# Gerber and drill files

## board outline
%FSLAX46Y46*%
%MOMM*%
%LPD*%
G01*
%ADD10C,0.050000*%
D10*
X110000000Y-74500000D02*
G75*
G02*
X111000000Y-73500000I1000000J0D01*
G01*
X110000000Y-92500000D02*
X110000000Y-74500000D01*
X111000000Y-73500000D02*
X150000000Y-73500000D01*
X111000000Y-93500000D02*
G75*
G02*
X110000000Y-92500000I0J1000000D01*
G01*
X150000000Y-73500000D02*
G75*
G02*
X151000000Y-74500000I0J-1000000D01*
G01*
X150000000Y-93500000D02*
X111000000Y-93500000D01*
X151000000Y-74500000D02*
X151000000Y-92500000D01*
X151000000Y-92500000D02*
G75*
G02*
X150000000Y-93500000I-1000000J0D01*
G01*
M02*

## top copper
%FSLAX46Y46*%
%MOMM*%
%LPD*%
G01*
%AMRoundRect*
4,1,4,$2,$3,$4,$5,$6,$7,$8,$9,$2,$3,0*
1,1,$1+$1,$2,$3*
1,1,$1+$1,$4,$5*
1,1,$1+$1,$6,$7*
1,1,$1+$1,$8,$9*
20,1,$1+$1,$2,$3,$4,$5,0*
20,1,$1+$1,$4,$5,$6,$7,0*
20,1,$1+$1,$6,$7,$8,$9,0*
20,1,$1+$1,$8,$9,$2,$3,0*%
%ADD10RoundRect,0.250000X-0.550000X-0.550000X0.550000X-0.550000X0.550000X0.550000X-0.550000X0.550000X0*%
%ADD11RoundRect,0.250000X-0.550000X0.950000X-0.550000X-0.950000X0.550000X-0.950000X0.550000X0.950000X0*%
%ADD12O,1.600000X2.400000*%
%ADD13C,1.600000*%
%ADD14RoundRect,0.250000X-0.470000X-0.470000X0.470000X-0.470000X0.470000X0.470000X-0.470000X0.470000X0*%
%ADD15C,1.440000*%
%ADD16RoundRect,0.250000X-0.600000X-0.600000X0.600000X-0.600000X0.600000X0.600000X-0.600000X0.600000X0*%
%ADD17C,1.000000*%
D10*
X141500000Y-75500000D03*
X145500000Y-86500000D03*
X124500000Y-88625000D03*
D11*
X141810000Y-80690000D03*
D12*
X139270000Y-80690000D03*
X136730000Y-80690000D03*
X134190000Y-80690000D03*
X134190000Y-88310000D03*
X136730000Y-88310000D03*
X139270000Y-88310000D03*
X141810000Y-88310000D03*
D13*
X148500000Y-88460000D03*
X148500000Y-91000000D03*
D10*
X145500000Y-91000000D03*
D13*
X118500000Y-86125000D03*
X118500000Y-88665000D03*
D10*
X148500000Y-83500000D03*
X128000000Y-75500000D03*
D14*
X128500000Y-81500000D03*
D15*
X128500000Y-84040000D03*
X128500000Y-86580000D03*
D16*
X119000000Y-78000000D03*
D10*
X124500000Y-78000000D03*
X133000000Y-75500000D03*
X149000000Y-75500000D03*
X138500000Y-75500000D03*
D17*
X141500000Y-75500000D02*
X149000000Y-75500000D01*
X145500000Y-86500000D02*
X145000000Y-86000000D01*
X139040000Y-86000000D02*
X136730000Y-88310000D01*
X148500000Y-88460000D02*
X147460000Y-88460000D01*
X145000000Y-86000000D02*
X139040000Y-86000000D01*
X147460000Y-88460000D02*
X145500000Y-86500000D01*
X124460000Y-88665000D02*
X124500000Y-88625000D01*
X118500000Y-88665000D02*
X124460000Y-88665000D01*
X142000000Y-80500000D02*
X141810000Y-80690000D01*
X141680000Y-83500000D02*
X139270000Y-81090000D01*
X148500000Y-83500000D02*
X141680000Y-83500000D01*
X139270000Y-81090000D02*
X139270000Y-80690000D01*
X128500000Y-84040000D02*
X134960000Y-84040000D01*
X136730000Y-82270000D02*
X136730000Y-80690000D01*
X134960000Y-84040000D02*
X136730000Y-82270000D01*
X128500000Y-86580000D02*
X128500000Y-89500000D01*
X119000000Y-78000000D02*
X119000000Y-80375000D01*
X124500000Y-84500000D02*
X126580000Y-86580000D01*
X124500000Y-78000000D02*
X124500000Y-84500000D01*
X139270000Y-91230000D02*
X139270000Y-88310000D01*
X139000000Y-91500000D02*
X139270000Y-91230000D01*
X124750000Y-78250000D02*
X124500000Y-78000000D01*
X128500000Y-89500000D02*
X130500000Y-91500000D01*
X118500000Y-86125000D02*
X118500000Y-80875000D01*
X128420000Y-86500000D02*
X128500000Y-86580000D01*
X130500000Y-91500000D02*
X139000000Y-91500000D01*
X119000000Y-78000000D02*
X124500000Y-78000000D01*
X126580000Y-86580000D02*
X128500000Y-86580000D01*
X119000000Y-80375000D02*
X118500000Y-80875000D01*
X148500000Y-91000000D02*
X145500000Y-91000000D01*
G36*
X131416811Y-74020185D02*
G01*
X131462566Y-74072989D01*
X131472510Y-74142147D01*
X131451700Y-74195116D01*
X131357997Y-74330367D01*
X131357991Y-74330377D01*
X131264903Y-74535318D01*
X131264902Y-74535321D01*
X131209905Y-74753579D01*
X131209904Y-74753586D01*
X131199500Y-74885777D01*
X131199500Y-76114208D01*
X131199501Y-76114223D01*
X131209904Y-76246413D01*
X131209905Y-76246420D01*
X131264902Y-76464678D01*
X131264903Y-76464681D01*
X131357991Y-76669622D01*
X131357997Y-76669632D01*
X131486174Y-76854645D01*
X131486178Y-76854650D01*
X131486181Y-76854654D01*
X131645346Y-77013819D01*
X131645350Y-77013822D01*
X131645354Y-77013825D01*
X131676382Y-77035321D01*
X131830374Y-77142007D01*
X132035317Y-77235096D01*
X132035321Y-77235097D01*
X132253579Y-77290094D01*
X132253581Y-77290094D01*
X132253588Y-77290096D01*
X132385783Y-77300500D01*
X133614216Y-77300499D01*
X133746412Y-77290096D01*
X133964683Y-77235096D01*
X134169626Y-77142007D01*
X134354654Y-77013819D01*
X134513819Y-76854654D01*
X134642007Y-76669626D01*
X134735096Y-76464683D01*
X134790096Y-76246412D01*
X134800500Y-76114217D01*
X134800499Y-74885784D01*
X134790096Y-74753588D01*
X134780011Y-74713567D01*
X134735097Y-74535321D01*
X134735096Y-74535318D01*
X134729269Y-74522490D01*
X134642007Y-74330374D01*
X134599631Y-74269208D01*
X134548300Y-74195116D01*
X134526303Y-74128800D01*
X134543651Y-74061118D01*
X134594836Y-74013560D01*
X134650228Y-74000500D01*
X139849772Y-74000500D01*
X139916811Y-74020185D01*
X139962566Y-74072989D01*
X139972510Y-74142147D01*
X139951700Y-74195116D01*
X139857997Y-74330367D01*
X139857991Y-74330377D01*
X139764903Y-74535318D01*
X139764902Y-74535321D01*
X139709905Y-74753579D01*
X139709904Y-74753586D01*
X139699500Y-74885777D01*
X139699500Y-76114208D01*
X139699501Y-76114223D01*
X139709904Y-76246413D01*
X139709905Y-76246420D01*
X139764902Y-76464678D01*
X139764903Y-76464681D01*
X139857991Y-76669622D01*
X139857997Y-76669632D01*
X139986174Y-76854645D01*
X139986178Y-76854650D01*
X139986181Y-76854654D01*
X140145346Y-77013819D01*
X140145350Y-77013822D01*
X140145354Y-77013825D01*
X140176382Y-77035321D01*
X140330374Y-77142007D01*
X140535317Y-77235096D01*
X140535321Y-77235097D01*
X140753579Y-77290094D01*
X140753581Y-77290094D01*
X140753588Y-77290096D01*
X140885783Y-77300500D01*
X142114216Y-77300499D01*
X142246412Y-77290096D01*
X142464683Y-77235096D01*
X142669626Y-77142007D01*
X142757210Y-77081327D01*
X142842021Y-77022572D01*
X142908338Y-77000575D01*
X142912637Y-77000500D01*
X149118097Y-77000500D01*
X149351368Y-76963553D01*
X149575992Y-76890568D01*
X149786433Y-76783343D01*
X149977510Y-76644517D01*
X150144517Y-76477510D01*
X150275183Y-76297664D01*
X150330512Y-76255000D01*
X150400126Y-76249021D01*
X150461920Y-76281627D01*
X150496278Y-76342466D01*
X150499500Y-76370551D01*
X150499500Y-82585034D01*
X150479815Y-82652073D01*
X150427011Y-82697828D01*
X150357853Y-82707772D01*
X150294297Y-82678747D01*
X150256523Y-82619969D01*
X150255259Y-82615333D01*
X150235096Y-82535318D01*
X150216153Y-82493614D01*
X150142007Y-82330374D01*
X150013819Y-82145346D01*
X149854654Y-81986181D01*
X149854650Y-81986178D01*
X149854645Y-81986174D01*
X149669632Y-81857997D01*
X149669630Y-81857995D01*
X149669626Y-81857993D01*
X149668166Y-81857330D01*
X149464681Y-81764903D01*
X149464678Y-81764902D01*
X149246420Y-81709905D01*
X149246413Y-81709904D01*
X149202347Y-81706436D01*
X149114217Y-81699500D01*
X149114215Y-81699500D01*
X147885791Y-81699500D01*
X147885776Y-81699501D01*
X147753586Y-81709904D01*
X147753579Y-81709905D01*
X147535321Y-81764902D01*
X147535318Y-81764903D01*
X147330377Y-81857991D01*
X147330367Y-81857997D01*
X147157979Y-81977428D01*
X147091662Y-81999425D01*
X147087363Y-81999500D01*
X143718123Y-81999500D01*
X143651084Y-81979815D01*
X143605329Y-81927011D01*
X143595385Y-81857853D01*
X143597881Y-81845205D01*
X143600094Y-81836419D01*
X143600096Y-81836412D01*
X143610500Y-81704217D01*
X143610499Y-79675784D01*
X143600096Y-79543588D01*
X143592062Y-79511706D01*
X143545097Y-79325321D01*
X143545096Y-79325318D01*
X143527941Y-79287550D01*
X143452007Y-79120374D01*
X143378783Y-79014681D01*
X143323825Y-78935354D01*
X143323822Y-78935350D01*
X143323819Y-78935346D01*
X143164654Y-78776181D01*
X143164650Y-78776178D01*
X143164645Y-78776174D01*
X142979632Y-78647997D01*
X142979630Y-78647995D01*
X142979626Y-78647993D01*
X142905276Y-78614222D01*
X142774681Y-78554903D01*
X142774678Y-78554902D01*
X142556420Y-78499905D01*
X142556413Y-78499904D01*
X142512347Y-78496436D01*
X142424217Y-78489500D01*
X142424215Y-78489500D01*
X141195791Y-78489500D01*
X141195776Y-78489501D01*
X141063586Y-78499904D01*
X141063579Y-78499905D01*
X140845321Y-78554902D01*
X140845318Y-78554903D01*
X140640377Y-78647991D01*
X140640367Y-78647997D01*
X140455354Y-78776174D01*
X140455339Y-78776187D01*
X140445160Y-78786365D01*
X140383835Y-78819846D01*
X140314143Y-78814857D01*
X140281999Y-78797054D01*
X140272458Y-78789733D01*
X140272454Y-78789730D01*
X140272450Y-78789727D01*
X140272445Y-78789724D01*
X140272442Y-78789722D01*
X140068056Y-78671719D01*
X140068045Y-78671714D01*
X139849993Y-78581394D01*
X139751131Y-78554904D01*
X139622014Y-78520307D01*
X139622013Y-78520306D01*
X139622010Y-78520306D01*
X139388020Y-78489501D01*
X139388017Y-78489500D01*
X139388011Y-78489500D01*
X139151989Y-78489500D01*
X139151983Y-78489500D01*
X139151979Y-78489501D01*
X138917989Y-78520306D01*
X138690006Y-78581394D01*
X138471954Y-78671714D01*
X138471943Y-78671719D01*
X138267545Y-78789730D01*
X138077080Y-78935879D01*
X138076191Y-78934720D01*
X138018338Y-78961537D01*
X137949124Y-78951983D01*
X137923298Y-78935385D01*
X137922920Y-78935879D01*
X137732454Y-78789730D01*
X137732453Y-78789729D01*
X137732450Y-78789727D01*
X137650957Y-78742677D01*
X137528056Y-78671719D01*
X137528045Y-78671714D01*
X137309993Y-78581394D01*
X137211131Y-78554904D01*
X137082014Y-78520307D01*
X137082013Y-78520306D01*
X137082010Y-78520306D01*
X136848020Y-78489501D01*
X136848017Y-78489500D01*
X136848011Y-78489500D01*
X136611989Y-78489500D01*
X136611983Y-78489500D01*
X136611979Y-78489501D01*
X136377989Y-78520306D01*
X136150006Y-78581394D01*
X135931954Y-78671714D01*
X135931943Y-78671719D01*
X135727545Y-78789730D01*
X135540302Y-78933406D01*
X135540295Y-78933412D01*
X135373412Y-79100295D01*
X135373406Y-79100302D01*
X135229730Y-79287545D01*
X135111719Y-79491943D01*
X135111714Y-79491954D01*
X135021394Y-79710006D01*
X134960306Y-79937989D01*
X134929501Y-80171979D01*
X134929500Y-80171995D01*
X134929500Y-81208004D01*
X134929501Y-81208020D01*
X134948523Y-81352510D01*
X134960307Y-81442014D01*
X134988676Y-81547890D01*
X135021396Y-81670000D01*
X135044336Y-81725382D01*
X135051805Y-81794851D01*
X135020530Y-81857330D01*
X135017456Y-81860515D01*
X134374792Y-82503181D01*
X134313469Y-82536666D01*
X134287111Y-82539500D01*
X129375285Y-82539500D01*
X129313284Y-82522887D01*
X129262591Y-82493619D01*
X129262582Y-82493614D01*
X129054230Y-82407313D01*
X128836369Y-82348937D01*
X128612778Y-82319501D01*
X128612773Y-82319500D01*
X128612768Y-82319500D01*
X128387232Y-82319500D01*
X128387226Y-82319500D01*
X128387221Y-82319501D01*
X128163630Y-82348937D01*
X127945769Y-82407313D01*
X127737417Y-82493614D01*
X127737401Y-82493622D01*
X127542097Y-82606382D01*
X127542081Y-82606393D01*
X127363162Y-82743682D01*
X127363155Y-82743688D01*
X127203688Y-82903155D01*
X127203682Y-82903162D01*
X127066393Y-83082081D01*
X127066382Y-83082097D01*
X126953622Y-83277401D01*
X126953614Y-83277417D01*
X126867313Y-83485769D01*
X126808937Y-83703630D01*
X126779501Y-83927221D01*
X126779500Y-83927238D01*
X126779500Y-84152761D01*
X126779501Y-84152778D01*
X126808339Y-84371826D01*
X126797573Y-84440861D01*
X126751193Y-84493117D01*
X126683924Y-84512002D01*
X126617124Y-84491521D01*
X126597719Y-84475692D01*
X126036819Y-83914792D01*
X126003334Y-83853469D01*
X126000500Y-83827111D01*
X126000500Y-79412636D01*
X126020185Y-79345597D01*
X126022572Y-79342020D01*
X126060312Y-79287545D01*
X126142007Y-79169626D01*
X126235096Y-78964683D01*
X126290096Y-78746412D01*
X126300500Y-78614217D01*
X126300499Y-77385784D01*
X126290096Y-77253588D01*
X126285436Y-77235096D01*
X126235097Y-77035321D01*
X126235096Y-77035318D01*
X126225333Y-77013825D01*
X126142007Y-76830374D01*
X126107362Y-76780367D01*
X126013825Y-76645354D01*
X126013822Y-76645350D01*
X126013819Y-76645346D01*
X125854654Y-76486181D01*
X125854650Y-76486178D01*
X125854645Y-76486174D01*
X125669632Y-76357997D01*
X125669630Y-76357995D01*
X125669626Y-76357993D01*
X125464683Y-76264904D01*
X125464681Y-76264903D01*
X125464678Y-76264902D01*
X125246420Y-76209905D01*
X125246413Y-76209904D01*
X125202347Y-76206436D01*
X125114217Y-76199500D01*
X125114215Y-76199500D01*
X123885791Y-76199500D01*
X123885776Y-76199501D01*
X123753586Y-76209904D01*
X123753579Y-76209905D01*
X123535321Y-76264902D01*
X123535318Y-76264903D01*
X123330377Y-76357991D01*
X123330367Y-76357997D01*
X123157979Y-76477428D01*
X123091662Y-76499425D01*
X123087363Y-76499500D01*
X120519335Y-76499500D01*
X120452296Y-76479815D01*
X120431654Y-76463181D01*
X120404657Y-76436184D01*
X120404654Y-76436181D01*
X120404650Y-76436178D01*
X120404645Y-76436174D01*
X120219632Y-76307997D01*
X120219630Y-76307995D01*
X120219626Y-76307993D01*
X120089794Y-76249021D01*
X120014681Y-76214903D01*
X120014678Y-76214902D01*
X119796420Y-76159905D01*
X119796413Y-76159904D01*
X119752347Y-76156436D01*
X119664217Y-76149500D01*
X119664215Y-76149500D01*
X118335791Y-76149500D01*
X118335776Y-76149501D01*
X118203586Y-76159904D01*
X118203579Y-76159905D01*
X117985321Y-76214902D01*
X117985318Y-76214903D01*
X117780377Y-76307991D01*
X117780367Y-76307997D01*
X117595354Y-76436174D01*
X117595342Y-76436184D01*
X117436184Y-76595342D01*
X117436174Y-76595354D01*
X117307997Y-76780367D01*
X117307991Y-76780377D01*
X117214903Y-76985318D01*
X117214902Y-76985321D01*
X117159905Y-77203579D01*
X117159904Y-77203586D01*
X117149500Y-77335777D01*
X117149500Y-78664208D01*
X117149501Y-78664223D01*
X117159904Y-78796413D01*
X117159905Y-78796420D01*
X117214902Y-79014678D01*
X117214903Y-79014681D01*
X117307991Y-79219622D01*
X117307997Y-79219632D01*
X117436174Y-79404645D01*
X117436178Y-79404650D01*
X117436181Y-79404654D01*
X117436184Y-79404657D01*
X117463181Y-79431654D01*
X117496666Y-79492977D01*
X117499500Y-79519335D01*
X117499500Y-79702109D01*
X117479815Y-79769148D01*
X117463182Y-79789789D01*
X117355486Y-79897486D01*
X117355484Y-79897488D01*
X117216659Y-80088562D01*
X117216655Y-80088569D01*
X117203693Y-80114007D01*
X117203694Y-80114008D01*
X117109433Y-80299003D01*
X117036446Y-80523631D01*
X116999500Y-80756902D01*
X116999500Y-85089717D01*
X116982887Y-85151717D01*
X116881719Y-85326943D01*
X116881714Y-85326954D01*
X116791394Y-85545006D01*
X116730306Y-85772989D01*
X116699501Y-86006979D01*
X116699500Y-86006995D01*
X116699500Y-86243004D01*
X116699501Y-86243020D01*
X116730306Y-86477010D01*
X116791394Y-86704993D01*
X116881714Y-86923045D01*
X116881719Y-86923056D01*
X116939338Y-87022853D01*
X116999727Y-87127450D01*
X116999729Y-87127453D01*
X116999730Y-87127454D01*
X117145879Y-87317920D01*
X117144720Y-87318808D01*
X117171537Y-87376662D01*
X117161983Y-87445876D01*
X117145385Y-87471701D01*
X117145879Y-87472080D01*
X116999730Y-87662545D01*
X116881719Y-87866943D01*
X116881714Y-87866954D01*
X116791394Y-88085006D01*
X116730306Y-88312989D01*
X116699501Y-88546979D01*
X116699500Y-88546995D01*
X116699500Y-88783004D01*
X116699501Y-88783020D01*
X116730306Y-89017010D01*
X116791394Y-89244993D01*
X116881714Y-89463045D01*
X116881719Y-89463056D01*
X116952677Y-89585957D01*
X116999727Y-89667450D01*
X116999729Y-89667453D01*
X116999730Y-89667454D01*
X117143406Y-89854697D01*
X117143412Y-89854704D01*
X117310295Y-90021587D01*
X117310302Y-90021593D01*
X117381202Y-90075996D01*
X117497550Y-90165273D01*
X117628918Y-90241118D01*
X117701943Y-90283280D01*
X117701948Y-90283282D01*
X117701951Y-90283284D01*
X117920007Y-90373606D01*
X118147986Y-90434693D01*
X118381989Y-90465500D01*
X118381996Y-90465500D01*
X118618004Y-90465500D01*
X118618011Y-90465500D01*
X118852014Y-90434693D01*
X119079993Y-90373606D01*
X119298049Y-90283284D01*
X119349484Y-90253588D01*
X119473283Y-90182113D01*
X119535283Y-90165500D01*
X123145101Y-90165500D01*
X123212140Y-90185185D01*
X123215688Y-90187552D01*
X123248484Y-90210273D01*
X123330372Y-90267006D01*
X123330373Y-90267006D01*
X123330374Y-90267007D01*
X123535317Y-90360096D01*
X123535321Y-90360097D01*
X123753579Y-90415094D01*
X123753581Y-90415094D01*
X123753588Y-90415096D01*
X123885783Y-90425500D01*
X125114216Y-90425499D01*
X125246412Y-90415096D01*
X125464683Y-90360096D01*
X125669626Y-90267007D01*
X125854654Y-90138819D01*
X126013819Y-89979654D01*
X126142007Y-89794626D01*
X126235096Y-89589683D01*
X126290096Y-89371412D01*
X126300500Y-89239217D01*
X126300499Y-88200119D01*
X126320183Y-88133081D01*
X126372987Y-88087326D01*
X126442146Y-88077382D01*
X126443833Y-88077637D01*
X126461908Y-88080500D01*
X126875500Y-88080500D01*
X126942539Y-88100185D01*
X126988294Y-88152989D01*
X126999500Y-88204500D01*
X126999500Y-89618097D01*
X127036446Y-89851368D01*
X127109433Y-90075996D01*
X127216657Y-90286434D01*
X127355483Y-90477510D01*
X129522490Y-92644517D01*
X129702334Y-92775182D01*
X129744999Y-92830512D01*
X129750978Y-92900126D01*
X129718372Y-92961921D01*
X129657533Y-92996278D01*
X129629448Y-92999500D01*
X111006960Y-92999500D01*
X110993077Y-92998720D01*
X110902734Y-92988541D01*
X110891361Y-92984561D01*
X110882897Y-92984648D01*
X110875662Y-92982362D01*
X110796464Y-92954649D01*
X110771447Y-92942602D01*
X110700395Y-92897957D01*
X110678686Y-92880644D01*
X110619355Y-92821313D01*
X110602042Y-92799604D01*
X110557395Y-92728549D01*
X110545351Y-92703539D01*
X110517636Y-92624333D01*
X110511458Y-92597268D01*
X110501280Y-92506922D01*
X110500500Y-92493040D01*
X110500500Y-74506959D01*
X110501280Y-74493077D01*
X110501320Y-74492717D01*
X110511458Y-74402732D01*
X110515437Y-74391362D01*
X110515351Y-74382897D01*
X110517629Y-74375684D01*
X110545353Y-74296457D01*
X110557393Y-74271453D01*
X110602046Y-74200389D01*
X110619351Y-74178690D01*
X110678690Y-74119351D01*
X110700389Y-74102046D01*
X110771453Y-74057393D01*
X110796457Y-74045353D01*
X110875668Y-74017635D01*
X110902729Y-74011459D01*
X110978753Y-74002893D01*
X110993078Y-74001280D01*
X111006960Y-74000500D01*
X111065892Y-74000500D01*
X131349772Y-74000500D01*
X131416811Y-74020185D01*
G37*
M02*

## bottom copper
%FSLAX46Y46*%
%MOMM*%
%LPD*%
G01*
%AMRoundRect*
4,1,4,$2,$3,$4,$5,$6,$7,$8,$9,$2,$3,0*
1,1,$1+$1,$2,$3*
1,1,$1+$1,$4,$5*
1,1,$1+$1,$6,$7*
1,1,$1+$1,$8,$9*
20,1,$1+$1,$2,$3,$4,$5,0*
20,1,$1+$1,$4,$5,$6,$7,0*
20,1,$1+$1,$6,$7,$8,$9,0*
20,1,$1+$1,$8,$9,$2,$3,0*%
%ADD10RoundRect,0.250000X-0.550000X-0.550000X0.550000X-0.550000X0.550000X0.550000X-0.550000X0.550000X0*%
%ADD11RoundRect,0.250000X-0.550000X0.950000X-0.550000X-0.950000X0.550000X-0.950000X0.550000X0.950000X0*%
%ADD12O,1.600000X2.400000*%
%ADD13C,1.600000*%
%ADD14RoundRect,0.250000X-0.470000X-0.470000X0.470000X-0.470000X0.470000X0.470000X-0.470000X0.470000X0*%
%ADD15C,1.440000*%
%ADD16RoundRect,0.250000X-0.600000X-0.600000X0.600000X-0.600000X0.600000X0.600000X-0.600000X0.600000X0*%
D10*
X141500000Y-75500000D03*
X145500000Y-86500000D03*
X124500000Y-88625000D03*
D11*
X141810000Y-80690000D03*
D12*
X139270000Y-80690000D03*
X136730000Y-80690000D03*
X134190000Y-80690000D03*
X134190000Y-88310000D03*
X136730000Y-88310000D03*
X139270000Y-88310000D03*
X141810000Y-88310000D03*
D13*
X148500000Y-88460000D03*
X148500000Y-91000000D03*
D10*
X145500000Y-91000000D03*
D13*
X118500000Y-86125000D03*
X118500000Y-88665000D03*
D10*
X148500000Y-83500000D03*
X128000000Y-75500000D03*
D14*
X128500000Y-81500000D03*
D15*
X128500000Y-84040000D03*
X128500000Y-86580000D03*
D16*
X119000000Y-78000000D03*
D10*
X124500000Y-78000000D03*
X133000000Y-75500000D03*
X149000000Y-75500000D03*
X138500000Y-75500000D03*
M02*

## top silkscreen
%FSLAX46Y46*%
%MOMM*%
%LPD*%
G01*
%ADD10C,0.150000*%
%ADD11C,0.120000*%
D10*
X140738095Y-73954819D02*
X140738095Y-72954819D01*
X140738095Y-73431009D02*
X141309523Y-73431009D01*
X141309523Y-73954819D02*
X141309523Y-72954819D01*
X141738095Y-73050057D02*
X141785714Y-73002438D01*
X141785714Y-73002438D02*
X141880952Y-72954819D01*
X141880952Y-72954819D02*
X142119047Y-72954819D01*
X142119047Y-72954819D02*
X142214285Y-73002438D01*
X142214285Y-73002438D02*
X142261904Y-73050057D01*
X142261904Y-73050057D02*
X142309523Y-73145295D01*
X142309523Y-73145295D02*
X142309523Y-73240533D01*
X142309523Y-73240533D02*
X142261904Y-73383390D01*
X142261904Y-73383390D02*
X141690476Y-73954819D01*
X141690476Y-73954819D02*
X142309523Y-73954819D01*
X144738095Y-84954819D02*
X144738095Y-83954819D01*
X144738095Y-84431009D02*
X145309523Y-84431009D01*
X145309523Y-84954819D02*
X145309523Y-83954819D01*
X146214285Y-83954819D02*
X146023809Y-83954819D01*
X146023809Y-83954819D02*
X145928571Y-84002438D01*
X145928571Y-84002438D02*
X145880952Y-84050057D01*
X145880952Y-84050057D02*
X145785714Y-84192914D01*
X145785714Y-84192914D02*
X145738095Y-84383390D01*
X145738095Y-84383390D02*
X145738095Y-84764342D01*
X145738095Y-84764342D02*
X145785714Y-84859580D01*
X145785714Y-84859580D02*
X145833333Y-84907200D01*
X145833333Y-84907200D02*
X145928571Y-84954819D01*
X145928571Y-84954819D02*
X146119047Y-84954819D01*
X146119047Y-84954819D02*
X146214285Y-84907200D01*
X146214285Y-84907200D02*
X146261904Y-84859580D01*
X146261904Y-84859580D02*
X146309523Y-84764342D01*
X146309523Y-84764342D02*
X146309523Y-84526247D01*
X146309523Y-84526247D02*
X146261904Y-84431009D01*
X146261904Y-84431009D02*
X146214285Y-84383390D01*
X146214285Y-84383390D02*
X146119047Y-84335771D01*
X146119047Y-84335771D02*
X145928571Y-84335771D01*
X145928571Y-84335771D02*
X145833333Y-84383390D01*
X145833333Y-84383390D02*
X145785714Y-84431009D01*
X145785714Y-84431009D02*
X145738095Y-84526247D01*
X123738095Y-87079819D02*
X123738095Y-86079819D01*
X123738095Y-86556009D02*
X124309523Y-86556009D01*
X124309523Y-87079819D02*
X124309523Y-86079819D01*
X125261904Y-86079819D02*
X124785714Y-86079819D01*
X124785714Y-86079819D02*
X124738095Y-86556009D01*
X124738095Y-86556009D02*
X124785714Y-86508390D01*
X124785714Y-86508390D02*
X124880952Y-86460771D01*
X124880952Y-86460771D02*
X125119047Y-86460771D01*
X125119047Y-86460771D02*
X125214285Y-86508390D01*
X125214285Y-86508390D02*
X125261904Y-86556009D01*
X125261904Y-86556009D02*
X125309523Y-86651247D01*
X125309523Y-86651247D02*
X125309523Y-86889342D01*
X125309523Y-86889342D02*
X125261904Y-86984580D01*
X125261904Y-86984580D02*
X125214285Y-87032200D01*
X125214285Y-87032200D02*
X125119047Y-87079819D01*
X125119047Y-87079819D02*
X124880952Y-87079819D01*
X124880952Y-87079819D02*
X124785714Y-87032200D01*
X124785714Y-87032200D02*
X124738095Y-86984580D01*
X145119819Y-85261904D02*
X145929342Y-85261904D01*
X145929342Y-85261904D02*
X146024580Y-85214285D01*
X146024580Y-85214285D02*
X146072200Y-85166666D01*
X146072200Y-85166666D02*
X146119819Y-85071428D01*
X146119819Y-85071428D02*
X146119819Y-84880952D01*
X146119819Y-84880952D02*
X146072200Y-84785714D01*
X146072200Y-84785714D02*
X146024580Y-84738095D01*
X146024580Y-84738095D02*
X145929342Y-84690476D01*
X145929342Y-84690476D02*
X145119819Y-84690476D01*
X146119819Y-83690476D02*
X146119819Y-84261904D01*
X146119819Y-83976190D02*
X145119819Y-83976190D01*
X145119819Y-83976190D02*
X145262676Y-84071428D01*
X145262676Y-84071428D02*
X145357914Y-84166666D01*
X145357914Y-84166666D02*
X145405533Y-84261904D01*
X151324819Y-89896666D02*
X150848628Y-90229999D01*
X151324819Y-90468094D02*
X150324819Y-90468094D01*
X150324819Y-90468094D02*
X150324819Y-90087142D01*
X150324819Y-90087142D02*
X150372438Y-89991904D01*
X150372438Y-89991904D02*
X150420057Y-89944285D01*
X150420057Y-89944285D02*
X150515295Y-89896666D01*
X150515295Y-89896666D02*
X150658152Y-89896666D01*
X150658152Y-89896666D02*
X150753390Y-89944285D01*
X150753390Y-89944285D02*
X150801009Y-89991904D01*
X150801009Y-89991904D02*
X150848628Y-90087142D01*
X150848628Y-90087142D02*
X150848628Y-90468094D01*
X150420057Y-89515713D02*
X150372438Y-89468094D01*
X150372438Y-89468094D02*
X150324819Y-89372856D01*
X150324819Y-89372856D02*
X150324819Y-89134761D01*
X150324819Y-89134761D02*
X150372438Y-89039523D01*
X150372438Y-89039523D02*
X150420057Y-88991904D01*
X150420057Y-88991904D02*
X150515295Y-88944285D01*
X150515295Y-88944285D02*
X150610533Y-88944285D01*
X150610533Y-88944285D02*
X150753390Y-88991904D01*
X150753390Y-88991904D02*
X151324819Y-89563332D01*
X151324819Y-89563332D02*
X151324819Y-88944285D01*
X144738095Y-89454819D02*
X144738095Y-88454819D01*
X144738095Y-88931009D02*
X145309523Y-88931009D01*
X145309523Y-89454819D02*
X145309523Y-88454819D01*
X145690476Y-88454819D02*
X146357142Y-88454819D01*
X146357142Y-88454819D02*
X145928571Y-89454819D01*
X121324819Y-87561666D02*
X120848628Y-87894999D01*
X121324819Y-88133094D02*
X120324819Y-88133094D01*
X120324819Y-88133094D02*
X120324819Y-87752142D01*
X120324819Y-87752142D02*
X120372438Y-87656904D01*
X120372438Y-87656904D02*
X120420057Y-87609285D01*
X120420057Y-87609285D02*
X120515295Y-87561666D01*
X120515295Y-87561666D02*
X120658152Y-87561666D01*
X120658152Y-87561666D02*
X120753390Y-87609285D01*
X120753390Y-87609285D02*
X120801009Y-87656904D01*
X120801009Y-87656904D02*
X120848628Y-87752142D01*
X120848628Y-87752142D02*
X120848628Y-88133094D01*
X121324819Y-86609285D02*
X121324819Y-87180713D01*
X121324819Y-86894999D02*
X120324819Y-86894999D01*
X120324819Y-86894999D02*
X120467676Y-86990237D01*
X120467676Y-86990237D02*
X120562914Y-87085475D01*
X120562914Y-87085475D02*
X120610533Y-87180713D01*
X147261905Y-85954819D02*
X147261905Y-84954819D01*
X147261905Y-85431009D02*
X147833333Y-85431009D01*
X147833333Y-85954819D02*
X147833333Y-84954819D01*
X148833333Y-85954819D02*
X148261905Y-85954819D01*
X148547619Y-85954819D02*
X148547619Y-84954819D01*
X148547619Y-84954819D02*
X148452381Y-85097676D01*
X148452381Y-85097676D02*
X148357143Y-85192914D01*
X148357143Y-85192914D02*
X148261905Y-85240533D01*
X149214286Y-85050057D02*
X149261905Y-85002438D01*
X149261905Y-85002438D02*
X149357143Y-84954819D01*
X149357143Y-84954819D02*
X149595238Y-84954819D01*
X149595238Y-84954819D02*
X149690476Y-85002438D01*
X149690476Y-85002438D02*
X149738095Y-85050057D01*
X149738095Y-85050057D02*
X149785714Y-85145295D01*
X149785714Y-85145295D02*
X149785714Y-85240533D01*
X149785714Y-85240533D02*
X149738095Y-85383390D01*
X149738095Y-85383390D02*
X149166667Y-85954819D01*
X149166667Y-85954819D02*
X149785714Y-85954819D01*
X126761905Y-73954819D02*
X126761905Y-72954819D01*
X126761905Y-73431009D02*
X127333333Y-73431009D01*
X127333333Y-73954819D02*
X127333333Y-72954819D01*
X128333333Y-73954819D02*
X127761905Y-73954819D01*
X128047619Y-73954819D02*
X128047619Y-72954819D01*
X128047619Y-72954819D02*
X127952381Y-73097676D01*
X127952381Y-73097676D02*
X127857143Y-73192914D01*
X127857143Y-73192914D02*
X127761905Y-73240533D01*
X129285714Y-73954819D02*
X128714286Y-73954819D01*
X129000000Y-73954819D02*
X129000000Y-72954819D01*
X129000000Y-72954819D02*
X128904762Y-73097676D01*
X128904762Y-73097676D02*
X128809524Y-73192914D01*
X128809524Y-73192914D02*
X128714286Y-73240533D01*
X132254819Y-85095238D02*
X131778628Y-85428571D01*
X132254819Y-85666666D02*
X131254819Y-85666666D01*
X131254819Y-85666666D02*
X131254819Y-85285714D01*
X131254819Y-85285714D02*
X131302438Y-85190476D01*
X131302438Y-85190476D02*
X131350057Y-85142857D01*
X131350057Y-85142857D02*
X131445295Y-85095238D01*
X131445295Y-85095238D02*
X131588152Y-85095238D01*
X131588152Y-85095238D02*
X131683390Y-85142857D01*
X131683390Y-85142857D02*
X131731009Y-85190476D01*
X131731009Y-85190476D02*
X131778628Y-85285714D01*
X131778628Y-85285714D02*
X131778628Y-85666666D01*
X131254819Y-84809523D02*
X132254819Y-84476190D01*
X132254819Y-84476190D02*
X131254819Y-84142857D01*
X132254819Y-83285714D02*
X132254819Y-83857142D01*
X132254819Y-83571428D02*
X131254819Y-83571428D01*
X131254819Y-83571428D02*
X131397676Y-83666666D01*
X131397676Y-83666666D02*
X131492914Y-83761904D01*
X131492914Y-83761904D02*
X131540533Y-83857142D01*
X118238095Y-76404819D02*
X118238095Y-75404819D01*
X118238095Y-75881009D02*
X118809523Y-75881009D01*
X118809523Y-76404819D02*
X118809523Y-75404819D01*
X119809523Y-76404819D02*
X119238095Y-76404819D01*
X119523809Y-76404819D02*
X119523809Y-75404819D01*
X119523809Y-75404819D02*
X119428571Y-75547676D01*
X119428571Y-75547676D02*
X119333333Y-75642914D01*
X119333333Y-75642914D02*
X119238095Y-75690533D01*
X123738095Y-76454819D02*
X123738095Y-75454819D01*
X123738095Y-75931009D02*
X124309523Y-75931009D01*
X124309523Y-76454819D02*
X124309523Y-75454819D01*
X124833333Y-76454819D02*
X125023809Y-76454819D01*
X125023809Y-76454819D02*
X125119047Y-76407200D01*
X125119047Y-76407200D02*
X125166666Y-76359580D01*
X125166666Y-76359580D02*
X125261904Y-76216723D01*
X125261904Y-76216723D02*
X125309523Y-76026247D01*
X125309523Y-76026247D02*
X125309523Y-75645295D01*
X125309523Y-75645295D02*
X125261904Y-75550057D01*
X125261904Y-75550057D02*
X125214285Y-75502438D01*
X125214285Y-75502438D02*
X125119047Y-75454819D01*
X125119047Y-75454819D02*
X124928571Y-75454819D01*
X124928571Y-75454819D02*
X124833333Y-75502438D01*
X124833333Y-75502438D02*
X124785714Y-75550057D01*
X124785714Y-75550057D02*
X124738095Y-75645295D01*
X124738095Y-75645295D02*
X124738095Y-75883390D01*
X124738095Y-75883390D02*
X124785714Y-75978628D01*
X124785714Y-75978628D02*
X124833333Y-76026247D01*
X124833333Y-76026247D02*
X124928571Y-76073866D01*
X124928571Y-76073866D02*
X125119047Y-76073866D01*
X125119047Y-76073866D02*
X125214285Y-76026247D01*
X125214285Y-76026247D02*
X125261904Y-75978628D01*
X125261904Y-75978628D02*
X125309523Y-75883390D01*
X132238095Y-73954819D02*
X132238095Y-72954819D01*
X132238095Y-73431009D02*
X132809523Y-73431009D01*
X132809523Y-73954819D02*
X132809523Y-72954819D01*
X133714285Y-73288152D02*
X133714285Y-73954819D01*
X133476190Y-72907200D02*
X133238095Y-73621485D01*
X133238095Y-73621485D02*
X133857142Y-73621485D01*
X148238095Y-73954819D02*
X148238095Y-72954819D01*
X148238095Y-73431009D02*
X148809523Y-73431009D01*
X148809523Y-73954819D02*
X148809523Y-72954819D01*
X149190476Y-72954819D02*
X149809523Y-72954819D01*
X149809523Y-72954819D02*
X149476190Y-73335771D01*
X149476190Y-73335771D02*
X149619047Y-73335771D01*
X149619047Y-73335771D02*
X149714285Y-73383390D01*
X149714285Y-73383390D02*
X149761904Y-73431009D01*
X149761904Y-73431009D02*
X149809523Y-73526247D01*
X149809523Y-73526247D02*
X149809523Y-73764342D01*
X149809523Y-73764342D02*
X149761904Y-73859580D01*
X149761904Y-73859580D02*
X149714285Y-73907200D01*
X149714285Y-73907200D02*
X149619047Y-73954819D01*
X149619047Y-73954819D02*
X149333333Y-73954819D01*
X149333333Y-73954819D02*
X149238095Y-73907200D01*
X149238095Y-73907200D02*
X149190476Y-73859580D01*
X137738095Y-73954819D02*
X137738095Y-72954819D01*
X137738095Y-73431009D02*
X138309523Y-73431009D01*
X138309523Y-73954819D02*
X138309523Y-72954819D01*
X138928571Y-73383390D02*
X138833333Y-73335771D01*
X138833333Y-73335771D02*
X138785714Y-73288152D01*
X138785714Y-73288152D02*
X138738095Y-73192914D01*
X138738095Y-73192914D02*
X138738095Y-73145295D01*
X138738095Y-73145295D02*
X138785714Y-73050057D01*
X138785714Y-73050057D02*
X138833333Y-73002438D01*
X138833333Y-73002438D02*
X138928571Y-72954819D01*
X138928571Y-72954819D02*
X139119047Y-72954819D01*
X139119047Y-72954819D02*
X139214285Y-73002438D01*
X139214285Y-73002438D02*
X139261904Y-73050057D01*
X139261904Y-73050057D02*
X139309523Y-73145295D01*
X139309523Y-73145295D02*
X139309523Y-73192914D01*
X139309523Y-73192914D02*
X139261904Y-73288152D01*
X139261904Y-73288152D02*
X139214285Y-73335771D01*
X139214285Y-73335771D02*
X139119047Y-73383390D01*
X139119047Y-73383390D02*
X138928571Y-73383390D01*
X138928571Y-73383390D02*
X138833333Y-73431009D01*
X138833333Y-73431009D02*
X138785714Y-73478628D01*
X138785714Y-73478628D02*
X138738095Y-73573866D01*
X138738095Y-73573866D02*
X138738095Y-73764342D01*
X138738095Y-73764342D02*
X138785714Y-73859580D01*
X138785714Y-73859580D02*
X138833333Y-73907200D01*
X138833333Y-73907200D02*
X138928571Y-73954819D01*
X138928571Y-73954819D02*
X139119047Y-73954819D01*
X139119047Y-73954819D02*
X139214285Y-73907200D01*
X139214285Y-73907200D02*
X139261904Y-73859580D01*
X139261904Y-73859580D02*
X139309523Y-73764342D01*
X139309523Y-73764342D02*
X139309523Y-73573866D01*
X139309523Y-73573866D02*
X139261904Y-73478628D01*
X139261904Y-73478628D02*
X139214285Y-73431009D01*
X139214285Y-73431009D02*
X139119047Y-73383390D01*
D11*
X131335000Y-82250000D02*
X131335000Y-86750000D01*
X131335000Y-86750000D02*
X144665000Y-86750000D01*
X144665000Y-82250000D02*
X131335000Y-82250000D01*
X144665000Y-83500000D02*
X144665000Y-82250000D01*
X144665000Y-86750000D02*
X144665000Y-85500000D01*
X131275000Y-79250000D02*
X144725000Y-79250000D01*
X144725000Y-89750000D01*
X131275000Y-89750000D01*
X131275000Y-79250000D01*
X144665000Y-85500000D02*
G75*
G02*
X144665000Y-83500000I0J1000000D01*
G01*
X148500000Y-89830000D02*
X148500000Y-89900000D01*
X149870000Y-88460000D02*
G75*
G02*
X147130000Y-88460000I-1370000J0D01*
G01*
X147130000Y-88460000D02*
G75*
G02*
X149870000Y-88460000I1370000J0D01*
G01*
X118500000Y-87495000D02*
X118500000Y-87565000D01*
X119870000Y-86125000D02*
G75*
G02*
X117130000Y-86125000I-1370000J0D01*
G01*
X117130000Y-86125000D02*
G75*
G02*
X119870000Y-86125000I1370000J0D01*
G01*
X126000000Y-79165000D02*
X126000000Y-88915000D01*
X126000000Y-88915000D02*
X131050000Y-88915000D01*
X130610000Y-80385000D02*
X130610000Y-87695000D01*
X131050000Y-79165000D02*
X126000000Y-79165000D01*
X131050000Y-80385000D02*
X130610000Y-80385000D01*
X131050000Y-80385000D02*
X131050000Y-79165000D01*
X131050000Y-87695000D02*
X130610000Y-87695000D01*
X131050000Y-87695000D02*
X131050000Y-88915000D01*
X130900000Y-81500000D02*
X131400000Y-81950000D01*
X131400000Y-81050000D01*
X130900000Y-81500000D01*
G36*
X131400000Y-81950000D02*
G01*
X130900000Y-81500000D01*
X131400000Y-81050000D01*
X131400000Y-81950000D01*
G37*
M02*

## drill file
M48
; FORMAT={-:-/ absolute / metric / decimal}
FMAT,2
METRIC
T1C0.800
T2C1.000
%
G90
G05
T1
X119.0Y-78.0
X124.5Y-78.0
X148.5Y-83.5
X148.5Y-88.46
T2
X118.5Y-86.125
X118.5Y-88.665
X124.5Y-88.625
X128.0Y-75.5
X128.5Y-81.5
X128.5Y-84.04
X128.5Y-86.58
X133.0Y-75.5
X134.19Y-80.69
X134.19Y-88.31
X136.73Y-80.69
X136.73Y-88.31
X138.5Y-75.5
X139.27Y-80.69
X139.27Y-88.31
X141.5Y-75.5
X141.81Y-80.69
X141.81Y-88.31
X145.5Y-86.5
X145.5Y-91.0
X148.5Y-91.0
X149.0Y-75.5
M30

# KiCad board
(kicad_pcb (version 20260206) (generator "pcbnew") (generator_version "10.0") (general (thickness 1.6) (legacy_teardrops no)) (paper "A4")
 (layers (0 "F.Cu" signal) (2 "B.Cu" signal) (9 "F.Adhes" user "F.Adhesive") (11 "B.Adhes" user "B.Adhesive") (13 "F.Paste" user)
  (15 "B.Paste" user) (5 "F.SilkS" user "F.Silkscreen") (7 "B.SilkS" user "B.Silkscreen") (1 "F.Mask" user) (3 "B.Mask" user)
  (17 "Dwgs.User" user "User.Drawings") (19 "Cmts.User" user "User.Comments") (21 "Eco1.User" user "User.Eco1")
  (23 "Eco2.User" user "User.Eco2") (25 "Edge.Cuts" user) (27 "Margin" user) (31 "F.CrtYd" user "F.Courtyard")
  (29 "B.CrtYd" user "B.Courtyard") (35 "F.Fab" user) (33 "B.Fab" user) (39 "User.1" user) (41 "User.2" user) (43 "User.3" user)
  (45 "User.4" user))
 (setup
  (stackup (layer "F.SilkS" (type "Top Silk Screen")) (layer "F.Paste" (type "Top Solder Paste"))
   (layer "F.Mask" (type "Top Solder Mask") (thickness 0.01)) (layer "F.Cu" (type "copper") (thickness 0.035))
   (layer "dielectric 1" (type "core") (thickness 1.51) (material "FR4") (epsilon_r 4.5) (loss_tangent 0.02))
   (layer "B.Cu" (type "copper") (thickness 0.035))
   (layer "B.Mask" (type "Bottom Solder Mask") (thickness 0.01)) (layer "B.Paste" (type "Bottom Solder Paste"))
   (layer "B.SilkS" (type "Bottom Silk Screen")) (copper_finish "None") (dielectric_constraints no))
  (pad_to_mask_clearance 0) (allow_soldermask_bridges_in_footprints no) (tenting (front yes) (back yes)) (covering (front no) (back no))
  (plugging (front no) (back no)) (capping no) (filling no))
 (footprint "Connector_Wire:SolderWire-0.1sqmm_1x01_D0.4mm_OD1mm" (layer "F.Cu") (at 141.5 75.5)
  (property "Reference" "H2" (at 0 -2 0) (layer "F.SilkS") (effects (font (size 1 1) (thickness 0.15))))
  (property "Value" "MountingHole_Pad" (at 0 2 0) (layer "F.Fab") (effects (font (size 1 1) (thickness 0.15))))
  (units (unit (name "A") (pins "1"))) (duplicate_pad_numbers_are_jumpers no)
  (pad "1" thru_hole roundrect (at 0 0) (size 1.6 1.6) (drill 1) (layers "*.Cu" "*.Mask") (remove_unused_layers no)
   (roundrect_rratio 0.15625) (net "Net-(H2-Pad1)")))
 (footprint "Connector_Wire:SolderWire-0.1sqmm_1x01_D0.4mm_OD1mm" (layer "F.Cu") (at 145.5 86.5)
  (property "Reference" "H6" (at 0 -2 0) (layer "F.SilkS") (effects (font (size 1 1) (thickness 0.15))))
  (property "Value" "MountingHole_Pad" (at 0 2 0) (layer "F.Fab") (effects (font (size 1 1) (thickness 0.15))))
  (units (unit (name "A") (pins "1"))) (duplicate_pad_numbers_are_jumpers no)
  (pad "1" thru_hole roundrect (at 0 0) (size 1.6 1.6) (drill 1) (layers "*.Cu" "*.Mask") (remove_unused_layers no)
   (roundrect_rratio 0.15625) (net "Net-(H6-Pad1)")))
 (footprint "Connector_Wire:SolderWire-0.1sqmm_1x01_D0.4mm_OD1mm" (layer "F.Cu") (at 124.5 88.625)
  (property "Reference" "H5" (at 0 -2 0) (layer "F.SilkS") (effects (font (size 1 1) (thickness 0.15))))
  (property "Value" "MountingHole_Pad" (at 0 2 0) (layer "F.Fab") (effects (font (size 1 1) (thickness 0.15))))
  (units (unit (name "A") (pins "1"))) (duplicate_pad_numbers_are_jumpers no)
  (pad "1" thru_hole roundrect (at 0 0) (size 1.6 1.6) (drill 1) (layers "*.Cu" "*.Mask") (remove_unused_layers no)
   (roundrect_rratio 0.15625) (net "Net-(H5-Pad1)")))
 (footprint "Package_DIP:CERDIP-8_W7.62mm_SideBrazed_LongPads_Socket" (layer "F.Cu") (at 141.81 80.69 -90)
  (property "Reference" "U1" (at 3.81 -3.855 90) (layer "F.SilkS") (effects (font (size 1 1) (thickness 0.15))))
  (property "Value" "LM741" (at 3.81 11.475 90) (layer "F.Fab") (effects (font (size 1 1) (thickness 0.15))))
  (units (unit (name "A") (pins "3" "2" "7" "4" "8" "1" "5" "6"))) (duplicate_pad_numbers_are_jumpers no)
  (fp_line (start 1.56 10.475) (end 6.06 10.475) (stroke (width 0.12) (type solid)) (layer "F.SilkS"))
  (fp_line (start 6.06 10.475) (end 6.06 -2.855) (stroke (width 0.12) (type solid)) (layer "F.SilkS"))
  (fp_line (start 1.56 -2.855) (end 1.56 10.475) (stroke (width 0.12) (type solid)) (layer "F.SilkS"))
  (fp_line (start 2.81 -2.855) (end 1.56 -2.855) (stroke (width 0.12) (type solid)) (layer "F.SilkS"))
  (fp_line (start 6.06 -2.855) (end 4.81 -2.855) (stroke (width 0.12) (type solid)) (layer "F.SilkS"))
  (fp_rect (start -1.44 -2.915) (end 9.06 10.535) (stroke (width 0.12) (type solid)) (fill no) (layer "F.SilkS"))
  (fp_arc (start 4.81 -2.855) (mid 3.81 -1.855) (end 2.81 -2.855) (stroke (width 0.12) (type solid)) (layer "F.SilkS"))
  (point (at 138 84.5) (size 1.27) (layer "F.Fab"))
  (pad "1" thru_hole roundrect (at 0 0 270) (size 2.4 1.6) (drill 1) (layers "*.Cu" "*.Mask") (remove_unused_layers no)
   (roundrect_rratio 0.15625) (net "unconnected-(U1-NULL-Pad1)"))
  (pad "2" thru_hole oval (at 0 2.54 270) (size 2.4 1.6) (drill 1) (layers "*.Cu" "*.Mask") (remove_unused_layers no) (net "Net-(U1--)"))
  (pad "3" thru_hole oval (at 0 5.08 270) (size 2.4 1.6) (drill 1) (layers "*.Cu" "*.Mask") (remove_unused_layers no) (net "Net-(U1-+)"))
  (pad "4" thru_hole oval (at 0 7.62 270) (size 2.4 1.6) (drill 1) (layers "*.Cu" "*.Mask") (remove_unused_layers no) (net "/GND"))
  (pad "5" thru_hole oval (at 7.62 7.62 270) (size 2.4 1.6) (drill 1) (layers "*.Cu" "*.Mask") (remove_unused_layers no)
   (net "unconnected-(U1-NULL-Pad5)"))
  (pad "6" thru_hole oval (at 7.62 5.08 270) (size 2.4 1.6) (drill 1) (layers "*.Cu" "*.Mask") (remove_unused_layers no)
   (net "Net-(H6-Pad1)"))
  (pad "7" thru_hole oval (at 7.62 2.54 270) (size 2.4 1.6) (drill 1) (layers "*.Cu" "*.Mask") (remove_unused_layers no) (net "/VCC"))
  (pad "8" thru_hole oval (at 7.62 0 270) (size 2.4 1.6) (drill 1) (layers "*.Cu" "*.Mask") (remove_unused_layers no)
   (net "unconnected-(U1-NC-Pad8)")))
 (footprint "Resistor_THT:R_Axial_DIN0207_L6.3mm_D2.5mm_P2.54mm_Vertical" (layer "F.Cu") (at 148.5 88.46 -90)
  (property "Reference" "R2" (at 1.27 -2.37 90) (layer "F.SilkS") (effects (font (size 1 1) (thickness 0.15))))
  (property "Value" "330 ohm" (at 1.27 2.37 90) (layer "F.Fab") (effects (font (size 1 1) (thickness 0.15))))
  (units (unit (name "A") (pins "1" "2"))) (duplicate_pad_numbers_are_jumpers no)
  (fp_line (start 1.37 0) (end 1.44 0) (stroke (width 0.12) (type solid)) (layer "F.SilkS"))
  (fp_circle (center 0 0) (end 1.37 0) (stroke (width 0.12) (type solid)) (fill no) (layer "F.SilkS"))
  (pad "1" thru_hole circle (at 0 0 270) (size 1.6 1.6) (drill 0.8) (layers "*.Cu" "*.Mask") (remove_unused_layers no) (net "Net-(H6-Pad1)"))
  (pad "2" thru_hole circle (at 2.54 0 270) (size 1.6 1.6) (drill 1) (layers "*.Cu" "*.Mask") (remove_unused_layers no)
   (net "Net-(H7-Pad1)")))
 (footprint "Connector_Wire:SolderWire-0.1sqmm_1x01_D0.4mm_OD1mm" (layer "F.Cu") (at 145.5 91)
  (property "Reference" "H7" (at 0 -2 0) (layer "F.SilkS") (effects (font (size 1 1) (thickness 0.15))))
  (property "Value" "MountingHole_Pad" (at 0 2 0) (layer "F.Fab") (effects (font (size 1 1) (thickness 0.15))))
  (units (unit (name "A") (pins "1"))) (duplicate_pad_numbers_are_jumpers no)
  (pad "1" thru_hole roundrect (at 0 0) (size 1.6 1.6) (drill 1) (layers "*.Cu" "*.Mask") (remove_unused_layers no)
   (roundrect_rratio 0.15625) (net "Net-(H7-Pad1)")))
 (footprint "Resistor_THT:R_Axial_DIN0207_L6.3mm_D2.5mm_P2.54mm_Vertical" (layer "F.Cu") (at 118.5 86.125 -90)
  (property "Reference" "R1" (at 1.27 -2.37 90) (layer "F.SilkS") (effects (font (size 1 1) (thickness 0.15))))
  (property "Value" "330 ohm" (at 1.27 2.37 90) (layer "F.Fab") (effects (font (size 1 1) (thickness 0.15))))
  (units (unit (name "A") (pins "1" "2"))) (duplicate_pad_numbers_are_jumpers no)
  (fp_line (start 1.37 0) (end 1.44 0) (stroke (width 0.12) (type solid)) (layer "F.SilkS"))
  (fp_circle (center 0 0) (end 1.37 0) (stroke (width 0.12) (type solid)) (fill no) (layer "F.SilkS"))
  (pad "1" thru_hole circle (at 0 0 270) (size 1.6 1.6) (drill 1) (layers "*.Cu" "*.Mask") (remove_unused_layers no) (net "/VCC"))
  (pad "2" thru_hole circle (at 2.54 0 270) (size 1.6 1.6) (drill 1) (layers "*.Cu" "*.Mask") (remove_unused_layers no)
   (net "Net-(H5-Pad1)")))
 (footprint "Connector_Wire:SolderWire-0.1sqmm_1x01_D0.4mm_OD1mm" (layer "F.Cu") (at 148.5 83.5)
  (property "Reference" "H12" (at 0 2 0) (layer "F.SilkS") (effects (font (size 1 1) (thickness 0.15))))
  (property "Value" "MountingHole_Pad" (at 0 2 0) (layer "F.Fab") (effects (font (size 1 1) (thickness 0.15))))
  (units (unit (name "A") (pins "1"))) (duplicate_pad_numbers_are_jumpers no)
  (pad "1" thru_hole roundrect (at 0 0) (size 1.6 1.6) (drill 0.8) (layers "*.Cu" "*.Mask") (remove_unused_layers no)
   (roundrect_rratio 0.15625) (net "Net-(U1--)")))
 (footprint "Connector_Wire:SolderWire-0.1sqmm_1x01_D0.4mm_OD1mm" (layer "F.Cu") (at 128 75.5)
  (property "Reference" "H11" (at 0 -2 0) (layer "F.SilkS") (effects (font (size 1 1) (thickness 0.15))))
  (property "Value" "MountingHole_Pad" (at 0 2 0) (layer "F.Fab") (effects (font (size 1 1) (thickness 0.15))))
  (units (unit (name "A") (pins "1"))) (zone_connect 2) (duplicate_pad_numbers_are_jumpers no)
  (pad "1" thru_hole roundrect (at 0 0) (size 1.6 1.6) (drill 1) (layers "*.Cu" "*.Mask") (remove_unused_layers no)
   (roundrect_rratio 0.15625) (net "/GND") (zone_connect 2)))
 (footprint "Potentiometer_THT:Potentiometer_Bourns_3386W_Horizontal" (layer "F.Cu") (at 128.5 81.5 -90)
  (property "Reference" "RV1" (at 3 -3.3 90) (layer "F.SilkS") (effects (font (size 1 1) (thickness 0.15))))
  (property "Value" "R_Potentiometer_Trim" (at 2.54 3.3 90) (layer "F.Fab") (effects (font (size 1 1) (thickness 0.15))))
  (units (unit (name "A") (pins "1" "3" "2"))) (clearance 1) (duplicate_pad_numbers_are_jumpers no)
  (fp_line (start -2.335 2.5) (end 7.415 2.5) (stroke (width 0.12) (type default)) (layer "F.SilkS"))
  (fp_line (start 7.415 2.5) (end 7.415 -2.55) (stroke (width 0.12) (type default)) (layer "F.SilkS"))
  (fp_line (start -1.115 -2.11) (end 6.195 -2.11) (stroke (width 0.12) (type default)) (layer "F.SilkS"))
  (fp_line (start -2.335 -2.55) (end -2.335 2.5) (stroke (width 0.12) (type default)) (layer "F.SilkS"))
  (fp_line (start -1.115 -2.55) (end -1.115 -2.11) (stroke (width 0.12) (type default)) (layer "F.SilkS"))
  (fp_line (start -1.115 -2.55) (end -2.335 -2.55) (stroke (width 0.12) (type default)) (layer "F.SilkS"))
  (fp_line (start 6.195 -2.55) (end 6.195 -2.11) (stroke (width 0.12) (type default)) (layer "F.SilkS"))
  (fp_line (start 6.195 -2.55) (end 7.415 -2.55) (stroke (width 0.12) (type default)) (layer "F.SilkS"))
  (fp_poly (pts (xy 0 -2.4) (xy 0.45 -2.9) (xy -0.45 -2.9)) (stroke (width 0.12) (type solid)) (fill yes) (layer "F.SilkS"))
  (pad "1" thru_hole roundrect (at 0 0) (size 1.44 1.44) (drill 1) (layers "*.Cu" "*.Mask") (remove_unused_layers no)
   (roundrect_rratio 0.1736111111) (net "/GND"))
  (pad "2" thru_hole circle (at 2.54 0) (size 1.44 1.44) (drill 1) (layers "*.Cu" "*.Mask") (remove_unused_layers no) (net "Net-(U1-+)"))
  (pad "3" thru_hole circle (at 5.08 0) (size 1.44 1.44) (drill 1) (layers "*.Cu" "*.Mask") (remove_unused_layers no) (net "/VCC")))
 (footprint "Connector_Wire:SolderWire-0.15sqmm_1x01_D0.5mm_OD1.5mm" (layer "F.Cu") (at 119 78)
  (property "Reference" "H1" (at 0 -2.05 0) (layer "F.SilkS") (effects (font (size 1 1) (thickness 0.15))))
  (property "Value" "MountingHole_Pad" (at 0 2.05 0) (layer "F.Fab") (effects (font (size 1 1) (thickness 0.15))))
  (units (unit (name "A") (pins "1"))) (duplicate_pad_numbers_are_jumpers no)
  (pad "1" thru_hole roundrect (at 0 0) (size 1.7 1.7) (drill 0.8) (layers "*.Cu" "*.Mask") (remove_unused_layers no)
   (roundrect_rratio 0.147059) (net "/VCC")))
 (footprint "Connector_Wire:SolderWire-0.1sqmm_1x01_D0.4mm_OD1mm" (layer "F.Cu") (at 124.5 78)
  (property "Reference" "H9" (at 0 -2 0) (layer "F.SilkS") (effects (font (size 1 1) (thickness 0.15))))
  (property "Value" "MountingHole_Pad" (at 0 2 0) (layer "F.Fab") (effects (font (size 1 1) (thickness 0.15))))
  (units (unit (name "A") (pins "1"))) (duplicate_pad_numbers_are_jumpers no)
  (pad "1" thru_hole roundrect (at 0 0) (size 1.6 1.6) (drill 0.8) (layers "*.Cu" "*.Mask") (remove_unused_layers no)
   (roundrect_rratio 0.15625) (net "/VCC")))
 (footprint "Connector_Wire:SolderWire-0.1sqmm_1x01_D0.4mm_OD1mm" (layer "F.Cu") (at 133 75.5)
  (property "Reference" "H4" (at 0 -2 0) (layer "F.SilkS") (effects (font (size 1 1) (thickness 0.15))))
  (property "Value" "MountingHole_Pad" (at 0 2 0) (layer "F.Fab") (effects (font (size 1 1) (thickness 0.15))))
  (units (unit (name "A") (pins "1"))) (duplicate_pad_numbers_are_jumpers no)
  (pad "1" thru_hole roundrect (at 0 0) (size 1.6 1.6) (drill 1) (layers "*.Cu" "*.Mask") (remove_unused_layers no)
   (roundrect_rratio 0.15625) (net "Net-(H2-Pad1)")))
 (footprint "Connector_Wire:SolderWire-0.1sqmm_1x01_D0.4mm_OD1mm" (layer "F.Cu") (at 149 75.5)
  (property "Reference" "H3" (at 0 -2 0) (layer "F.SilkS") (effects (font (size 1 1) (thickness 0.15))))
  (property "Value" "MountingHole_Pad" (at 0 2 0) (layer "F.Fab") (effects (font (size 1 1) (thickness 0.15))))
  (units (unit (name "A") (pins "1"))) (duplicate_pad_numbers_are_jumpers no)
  (pad "1" thru_hole roundrect (at 0 0) (size 1.6 1.6) (drill 1) (layers "*.Cu" "*.Mask") (remove_unused_layers no)
   (roundrect_rratio 0.15625) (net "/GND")))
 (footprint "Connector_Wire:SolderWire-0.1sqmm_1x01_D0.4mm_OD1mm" (layer "F.Cu") (at 138.5 75.5)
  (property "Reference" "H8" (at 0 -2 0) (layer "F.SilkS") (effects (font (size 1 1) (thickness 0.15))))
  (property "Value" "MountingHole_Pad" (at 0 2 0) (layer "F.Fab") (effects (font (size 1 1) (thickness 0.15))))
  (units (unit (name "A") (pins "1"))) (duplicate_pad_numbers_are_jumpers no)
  (pad "1" thru_hole roundrect (at 0 0) (size 1.6 1.6) (drill 1) (layers "*.Cu" "*.Mask") (remove_unused_layers no)
   (roundrect_rratio 0.15625) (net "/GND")))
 (gr_arc (start 110 74.5) (mid 110.292893 73.792893) (end 111 73.5) (stroke (width 0.05) (type default)) (layer "Edge.Cuts"))
 (gr_line (start 110 92.5) (end 110 74.5) (stroke (width 0.05) (type default)) (layer "Edge.Cuts"))
 (gr_line (start 111 73.5) (end 150 73.5) (stroke (width 0.05) (type default)) (layer "Edge.Cuts"))
 (gr_arc (start 111 93.5) (mid 110.292893 93.207107) (end 110 92.5) (stroke (width 0.05) (type default)) (layer "Edge.Cuts"))
 (gr_arc (start 150 73.5) (mid 150.707107 73.792893) (end 151 74.5) (stroke (width 0.05) (type default)) (layer "Edge.Cuts"))
 (gr_line (start 150 93.5) (end 111 93.5) (stroke (width 0.05) (type default)) (layer "Edge.Cuts"))
 (gr_line (start 151 74.5) (end 151 92.5) (stroke (width 0.05) (type default)) (layer "Edge.Cuts"))
 (gr_arc (start 151 92.5) (mid 150.707107 93.207107) (end 150 93.5) (stroke (width 0.05) (type default)) (layer "Edge.Cuts"))
 (segment (start 141.5 75.5) (end 149 75.5) (width 1) (layer "F.Cu") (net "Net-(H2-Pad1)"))
 (segment (start 145.5 86.5) (end 145 86) (width 1) (layer "F.Cu") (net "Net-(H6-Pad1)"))
 (segment (start 139.04 86) (end 136.73 88.31) (width 1) (layer "F.Cu") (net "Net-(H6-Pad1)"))
 (segment (start 148.5 88.46) (end 147.46 88.46) (width 1) (layer "F.Cu") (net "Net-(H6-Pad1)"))
 (segment (start 145 86) (end 139.04 86) (width 1) (layer "F.Cu") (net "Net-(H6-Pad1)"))
 (segment (start 147.46 88.46) (end 145.5 86.5) (width 1) (layer "F.Cu") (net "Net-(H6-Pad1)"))
 (segment (start 124.46 88.665) (end 124.5 88.625) (width 1) (layer "F.Cu") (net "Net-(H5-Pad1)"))
 (segment (start 118.5 88.665) (end 124.46 88.665) (width 1) (layer "F.Cu") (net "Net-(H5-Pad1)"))
 (segment (start 142 80.5) (end 141.81 80.69) (width 1) (layer "F.Cu") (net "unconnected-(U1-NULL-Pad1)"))
 (segment (start 141.68 83.5) (end 139.27 81.09) (width 1) (layer "F.Cu") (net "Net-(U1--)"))
 (segment (start 148.5 83.5) (end 141.68 83.5) (width 1) (layer "F.Cu") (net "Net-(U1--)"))
 (segment (start 139.27 81.09) (end 139.27 80.69) (width 1) (layer "F.Cu") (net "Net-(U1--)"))
 (segment (start 128.5 84.04) (end 134.96 84.04) (width 1) (layer "F.Cu") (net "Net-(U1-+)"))
 (segment (start 136.73 82.27) (end 136.73 80.69) (width 1) (layer "F.Cu") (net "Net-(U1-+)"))
 (segment (start 134.96 84.04) (end 136.73 82.27) (width 1) (layer "F.Cu") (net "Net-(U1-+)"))
 (segment (start 128.5 86.58) (end 128.5 89.5) (width 1) (layer "F.Cu") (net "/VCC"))
 (segment (start 119 78) (end 119 80.375) (width 1) (layer "F.Cu") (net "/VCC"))
 (segment (start 124.5 84.5) (end 126.58 86.58) (width 1) (layer "F.Cu") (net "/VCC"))
 (segment (start 124.5 78) (end 124.5 84.5) (width 1) (layer "F.Cu") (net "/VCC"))
 (segment (start 139.27 91.23) (end 139.27 88.31) (width 1) (layer "F.Cu") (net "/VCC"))
 (segment (start 139 91.5) (end 139.27 91.23) (width 1) (layer "F.Cu") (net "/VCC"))
 (segment (start 124.75 78.25) (end 124.5 78) (width 1) (layer "F.Cu") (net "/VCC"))
 (segment (start 128.5 89.5) (end 130.5 91.5) (width 1) (layer "F.Cu") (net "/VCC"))
 (segment (start 118.5 86.125) (end 118.5 80.875) (width 1) (layer "F.Cu") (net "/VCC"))
 (segment (start 128.42 86.5) (end 128.5 86.58) (width 1) (layer "F.Cu") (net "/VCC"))
 (segment (start 130.5 91.5) (end 139 91.5) (width 1) (layer "F.Cu") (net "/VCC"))
 (segment (start 119 78) (end 124.5 78) (width 1) (layer "F.Cu") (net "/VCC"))
 (segment (start 126.58 86.58) (end 128.5 86.58) (width 1) (layer "F.Cu") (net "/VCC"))
 (segment (start 119 80.375) (end 118.5 80.875) (width 1) (layer "F.Cu") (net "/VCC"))
 (segment (start 148.5 91) (end 145.5 91) (width 1) (layer "F.Cu") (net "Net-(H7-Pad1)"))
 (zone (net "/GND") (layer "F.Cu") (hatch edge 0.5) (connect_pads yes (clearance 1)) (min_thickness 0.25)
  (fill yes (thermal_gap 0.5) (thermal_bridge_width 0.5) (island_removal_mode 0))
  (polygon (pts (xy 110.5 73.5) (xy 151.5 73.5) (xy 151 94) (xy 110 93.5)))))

